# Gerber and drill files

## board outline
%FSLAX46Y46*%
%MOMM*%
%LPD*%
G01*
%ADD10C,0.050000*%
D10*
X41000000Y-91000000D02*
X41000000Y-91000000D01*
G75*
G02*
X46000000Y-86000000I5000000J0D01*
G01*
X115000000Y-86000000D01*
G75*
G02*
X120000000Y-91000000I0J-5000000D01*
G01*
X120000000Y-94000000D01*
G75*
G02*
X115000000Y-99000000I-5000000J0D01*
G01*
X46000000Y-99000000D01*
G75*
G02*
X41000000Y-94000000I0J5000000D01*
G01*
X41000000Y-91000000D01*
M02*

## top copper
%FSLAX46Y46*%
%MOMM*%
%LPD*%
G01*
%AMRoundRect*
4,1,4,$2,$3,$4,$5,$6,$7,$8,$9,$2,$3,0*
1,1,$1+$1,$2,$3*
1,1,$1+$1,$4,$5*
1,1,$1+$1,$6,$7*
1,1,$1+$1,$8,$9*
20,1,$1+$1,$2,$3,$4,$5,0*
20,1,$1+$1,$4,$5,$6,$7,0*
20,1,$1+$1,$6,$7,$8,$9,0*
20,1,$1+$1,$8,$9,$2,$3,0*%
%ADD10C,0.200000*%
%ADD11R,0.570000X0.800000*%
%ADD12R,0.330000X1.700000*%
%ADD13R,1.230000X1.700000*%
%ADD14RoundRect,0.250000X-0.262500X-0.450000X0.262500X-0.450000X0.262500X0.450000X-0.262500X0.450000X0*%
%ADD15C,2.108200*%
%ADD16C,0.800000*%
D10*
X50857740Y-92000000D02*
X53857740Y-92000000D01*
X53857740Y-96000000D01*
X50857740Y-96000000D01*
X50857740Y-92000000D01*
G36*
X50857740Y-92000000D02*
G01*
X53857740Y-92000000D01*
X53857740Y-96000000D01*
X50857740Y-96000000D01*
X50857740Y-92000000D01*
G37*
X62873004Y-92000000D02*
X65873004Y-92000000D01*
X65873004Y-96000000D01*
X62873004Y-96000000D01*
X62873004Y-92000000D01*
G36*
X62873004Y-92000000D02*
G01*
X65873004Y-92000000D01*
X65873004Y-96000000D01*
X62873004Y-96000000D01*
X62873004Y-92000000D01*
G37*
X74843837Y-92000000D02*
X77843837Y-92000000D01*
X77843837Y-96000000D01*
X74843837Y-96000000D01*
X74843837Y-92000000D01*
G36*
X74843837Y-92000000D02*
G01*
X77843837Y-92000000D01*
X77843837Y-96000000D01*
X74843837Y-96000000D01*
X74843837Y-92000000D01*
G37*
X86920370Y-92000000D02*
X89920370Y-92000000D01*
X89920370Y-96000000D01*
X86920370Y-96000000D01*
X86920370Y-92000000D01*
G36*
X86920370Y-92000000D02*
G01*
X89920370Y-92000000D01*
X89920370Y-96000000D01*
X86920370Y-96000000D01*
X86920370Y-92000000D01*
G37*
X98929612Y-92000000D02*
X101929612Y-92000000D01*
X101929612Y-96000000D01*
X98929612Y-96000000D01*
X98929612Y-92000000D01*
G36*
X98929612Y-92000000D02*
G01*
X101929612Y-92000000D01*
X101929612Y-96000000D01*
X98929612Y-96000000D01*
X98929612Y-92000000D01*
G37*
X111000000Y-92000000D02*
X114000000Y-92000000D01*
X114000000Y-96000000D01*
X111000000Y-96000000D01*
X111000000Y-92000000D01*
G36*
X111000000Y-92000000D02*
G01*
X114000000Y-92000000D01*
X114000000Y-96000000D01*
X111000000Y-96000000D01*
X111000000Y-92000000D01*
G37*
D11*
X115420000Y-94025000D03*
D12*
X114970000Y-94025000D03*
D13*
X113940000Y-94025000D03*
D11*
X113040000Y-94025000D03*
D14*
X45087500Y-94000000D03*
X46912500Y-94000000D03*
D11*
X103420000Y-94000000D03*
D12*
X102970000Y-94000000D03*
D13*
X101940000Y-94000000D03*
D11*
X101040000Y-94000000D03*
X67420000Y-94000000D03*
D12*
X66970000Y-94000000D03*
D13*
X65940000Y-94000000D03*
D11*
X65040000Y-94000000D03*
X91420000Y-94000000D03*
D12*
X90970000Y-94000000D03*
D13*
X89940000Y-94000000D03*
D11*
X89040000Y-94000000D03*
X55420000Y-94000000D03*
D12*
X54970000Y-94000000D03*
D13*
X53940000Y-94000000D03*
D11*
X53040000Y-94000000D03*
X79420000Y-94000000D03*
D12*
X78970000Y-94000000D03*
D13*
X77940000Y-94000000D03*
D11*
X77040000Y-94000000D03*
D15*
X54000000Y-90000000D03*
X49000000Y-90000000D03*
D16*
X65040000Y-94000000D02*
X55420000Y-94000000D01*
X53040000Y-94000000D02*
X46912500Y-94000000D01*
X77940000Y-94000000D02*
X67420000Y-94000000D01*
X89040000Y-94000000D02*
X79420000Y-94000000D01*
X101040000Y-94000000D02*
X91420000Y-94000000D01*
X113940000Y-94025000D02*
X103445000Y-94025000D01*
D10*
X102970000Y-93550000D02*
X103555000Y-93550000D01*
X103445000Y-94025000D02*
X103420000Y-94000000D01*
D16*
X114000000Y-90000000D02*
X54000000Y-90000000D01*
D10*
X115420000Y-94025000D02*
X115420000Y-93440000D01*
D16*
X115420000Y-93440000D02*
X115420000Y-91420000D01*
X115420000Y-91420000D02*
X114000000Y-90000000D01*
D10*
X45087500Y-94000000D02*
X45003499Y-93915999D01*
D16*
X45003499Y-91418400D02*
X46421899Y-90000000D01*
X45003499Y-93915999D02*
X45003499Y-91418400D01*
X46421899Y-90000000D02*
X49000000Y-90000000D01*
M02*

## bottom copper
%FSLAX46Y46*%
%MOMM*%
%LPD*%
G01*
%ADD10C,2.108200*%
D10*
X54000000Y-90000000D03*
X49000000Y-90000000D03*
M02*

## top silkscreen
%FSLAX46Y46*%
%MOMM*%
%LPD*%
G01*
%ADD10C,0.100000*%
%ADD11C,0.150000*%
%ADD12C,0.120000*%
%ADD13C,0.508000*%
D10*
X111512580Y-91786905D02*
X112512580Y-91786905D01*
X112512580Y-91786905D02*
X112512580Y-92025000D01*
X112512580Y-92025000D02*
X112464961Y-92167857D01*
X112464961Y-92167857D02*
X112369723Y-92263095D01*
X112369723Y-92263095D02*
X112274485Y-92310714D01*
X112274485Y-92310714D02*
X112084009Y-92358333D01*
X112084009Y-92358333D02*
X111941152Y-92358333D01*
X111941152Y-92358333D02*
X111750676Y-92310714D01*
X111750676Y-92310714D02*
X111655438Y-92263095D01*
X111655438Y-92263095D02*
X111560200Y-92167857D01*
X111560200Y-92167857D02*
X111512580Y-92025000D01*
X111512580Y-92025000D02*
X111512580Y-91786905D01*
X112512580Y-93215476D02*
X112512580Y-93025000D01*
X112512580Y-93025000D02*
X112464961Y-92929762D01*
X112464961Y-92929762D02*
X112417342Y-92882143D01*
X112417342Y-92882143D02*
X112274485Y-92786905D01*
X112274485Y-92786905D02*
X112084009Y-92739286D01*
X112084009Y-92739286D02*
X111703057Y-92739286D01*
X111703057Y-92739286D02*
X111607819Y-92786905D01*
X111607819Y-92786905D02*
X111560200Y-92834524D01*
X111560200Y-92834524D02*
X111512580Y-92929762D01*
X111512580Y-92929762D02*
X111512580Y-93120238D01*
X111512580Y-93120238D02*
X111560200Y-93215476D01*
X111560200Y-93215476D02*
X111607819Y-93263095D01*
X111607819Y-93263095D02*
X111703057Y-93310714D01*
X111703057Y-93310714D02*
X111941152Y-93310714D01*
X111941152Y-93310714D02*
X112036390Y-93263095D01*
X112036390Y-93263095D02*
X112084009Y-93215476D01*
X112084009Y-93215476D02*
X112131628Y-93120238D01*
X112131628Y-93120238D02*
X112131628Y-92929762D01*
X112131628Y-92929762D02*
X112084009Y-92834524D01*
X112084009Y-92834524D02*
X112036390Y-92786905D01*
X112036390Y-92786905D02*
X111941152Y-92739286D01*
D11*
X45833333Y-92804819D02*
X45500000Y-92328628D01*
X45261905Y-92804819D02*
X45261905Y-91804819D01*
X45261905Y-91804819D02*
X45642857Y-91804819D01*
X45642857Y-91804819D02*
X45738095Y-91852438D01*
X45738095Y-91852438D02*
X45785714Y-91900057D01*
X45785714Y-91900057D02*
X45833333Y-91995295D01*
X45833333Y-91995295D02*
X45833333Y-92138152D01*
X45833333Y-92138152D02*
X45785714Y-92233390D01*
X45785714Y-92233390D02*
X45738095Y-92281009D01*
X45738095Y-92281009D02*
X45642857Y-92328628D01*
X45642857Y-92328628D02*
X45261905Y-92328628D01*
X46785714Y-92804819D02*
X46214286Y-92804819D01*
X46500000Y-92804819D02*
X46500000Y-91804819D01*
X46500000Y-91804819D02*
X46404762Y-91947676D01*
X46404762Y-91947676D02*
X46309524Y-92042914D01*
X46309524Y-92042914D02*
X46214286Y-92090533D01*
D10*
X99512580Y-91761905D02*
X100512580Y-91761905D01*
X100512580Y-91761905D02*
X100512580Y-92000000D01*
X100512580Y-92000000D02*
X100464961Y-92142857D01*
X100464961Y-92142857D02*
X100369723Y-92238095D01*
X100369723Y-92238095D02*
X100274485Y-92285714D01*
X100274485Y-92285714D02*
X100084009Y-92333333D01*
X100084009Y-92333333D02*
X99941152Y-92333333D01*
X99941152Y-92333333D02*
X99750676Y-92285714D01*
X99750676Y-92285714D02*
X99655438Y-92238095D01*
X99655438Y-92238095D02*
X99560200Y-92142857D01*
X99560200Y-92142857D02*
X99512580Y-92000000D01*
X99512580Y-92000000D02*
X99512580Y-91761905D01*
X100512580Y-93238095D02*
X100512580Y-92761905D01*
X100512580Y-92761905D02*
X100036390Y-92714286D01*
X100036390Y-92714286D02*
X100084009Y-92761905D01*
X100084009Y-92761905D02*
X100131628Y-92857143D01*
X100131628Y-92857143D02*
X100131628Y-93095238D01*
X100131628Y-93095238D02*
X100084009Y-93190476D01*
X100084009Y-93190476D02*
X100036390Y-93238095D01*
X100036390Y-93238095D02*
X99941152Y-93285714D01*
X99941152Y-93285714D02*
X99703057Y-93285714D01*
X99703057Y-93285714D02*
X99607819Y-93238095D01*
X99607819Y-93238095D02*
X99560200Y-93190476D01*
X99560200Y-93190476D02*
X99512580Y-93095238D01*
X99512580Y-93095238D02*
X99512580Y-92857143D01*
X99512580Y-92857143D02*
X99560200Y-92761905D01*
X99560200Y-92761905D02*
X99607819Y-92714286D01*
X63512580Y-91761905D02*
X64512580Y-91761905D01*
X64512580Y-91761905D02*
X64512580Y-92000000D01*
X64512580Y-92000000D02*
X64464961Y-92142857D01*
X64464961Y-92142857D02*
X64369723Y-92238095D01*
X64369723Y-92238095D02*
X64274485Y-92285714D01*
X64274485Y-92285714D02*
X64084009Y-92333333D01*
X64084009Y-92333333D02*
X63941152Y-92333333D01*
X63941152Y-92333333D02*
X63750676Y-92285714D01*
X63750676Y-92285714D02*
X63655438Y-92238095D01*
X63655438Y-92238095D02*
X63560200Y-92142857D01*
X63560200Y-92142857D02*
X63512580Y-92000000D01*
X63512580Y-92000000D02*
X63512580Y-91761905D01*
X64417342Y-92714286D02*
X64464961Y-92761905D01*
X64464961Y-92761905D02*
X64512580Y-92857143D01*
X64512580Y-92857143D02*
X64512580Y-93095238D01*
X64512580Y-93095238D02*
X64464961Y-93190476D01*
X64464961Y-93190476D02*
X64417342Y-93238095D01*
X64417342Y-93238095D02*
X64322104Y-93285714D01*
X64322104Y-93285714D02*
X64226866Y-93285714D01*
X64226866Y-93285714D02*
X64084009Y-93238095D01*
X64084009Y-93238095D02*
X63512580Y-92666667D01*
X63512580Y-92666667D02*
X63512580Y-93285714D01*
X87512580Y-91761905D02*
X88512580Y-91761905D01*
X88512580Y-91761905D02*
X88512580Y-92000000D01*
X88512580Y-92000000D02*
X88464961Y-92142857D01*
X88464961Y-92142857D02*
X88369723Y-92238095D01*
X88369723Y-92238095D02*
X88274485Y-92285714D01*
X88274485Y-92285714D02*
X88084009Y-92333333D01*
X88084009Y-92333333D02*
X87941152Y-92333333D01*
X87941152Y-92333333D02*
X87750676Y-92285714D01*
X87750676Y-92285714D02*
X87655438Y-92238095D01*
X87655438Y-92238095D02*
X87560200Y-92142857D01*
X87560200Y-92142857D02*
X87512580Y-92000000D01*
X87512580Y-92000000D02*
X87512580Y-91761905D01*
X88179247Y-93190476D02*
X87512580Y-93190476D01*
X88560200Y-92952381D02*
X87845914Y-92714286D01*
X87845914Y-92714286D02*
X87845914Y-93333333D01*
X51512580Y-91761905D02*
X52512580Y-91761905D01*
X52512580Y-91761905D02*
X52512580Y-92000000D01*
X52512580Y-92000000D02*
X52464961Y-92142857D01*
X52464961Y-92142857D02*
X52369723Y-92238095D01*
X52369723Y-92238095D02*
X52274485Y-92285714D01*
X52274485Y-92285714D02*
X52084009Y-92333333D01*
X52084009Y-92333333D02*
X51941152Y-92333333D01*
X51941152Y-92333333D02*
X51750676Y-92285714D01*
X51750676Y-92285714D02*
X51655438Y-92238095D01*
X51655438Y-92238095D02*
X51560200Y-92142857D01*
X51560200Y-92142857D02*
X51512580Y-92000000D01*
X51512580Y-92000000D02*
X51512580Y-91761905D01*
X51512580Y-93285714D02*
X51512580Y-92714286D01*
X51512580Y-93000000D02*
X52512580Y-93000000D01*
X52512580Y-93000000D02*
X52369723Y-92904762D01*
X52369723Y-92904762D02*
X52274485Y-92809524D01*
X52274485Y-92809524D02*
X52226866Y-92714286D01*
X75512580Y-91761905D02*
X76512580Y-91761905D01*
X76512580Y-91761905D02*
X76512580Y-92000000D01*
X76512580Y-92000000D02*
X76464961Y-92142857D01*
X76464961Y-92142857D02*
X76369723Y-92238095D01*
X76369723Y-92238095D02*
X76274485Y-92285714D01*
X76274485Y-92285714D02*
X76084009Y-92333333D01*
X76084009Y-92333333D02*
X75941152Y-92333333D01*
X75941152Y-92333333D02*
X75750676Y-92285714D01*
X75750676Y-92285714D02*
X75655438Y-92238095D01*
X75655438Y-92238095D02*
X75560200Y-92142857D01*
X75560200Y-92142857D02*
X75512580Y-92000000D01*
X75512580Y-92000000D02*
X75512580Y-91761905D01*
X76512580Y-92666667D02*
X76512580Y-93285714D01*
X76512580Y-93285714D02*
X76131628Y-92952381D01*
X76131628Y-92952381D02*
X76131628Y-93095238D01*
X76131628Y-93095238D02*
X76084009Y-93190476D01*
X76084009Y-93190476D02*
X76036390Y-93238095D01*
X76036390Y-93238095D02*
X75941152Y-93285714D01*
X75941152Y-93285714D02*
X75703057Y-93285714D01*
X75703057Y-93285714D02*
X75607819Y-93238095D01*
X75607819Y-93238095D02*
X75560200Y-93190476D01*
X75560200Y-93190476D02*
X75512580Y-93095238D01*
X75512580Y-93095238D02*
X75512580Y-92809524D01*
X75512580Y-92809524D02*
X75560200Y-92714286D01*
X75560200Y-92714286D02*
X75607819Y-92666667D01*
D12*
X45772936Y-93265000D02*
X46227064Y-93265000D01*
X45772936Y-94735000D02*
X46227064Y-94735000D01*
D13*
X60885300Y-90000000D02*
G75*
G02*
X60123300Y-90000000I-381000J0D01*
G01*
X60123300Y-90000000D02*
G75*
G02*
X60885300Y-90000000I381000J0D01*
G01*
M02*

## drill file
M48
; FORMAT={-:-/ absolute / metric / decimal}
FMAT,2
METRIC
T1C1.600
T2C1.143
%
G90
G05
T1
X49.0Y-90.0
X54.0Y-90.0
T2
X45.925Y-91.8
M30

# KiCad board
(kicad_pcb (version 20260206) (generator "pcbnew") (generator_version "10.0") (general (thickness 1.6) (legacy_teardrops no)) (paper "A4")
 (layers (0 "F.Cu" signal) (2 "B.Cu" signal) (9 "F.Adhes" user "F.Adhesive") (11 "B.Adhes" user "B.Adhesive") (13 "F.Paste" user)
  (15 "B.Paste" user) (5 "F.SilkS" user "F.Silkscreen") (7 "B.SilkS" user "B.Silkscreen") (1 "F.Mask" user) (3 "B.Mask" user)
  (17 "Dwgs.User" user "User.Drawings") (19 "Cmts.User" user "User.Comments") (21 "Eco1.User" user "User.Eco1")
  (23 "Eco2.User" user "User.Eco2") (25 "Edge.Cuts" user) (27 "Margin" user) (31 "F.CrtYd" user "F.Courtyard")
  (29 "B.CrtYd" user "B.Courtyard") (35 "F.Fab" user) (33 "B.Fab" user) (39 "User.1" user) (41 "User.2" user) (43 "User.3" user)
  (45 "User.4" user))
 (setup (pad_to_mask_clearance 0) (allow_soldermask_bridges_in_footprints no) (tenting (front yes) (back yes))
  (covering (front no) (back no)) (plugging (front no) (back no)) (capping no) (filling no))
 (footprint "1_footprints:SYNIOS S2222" (layer "F.Cu") (at 114.97 94.025 -90)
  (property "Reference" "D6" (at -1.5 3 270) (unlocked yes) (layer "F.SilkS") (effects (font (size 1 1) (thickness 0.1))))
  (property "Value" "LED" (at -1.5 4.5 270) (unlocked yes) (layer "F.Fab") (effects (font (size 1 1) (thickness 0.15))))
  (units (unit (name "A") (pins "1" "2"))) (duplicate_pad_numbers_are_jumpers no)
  (pad "1" smd rect (at 0 -0.45 270) (size 0.8 0.57) (layers "F.Cu" "F.Mask" "F.Paste") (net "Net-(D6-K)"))
  (pad "1" smd rect (at 0 0 270) (size 1.7 0.33) (layers "F.Cu" "F.Mask" "F.Paste") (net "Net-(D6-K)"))
  (pad "2" smd rect (at 0 1.03 270) (size 1.7 1.23) (layers "F.Cu" "F.Mask" "F.Paste") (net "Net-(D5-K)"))
  (pad "2" smd rect (at 0 1.93 270) (size 0.8 0.57) (layers "F.Cu" "F.Mask" "F.Paste") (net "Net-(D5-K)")))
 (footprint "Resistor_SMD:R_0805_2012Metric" (layer "F.Cu") (at 46 94)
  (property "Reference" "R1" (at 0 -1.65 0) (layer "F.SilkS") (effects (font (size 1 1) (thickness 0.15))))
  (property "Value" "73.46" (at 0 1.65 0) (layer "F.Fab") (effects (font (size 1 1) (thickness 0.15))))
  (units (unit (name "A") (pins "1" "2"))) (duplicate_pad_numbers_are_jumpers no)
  (fp_line (start -0.227064 -0.735) (end 0.227064 -0.735) (stroke (width 0.12) (type solid)) (layer "F.SilkS"))
  (fp_line (start -0.227064 0.735) (end 0.227064 0.735) (stroke (width 0.12) (type solid)) (layer "F.SilkS"))
  (pad "1" smd roundrect (at -0.9125 0) (size 1.025 1.4) (layers "F.Cu" "F.Mask" "F.Paste") (roundrect_rratio 0.243902)
   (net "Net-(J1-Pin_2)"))
  (pad "2" smd roundrect (at 0.9125 0) (size 1.025 1.4) (layers "F.Cu" "F.Mask" "F.Paste") (roundrect_rratio 0.243902) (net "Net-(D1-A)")))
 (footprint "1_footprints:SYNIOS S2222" (layer "F.Cu") (at 102.97 94 -90)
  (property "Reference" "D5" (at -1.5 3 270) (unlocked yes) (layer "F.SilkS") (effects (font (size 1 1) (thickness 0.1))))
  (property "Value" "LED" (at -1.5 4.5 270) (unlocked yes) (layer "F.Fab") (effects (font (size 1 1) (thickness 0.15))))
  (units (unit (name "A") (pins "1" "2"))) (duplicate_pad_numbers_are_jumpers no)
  (pad "1" smd rect (at 0 -0.45 270) (size 0.8 0.57) (layers "F.Cu" "F.Mask" "F.Paste") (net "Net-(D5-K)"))
  (pad "1" smd rect (at 0 0 270) (size 1.7 0.33) (layers "F.Cu" "F.Mask" "F.Paste") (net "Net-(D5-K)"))
  (pad "2" smd rect (at 0 1.03 270) (size 1.7 1.23) (layers "F.Cu" "F.Mask" "F.Paste") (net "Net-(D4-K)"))
  (pad "2" smd rect (at 0 1.93 270) (size 0.8 0.57) (layers "F.Cu" "F.Mask" "F.Paste") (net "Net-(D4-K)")))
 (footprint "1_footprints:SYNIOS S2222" (layer "F.Cu") (at 66.97 94 -90)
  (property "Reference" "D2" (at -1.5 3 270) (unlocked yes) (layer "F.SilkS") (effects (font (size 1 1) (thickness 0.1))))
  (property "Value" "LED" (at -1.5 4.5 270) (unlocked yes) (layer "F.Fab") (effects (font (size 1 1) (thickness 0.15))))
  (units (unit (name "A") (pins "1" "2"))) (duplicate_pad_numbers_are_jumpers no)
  (pad "1" smd rect (at 0 -0.45 270) (size 0.8 0.57) (layers "F.Cu" "F.Mask" "F.Paste") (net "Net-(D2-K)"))
  (pad "1" smd rect (at 0 0 270) (size 1.7 0.33) (layers "F.Cu" "F.Mask" "F.Paste") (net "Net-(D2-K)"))
  (pad "2" smd rect (at 0 1.03 270) (size 1.7 1.23) (layers "F.Cu" "F.Mask" "F.Paste") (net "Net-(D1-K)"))
  (pad "2" smd rect (at 0 1.93 270) (size 0.8 0.57) (layers "F.Cu" "F.Mask" "F.Paste") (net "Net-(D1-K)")))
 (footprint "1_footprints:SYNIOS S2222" (layer "F.Cu") (at 90.97 94 -90)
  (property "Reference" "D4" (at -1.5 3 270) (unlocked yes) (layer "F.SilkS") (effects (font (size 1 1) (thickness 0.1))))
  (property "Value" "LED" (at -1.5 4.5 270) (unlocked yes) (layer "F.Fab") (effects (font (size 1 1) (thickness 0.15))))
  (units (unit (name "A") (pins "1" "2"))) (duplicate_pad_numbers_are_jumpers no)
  (pad "1" smd rect (at 0 -0.45 270) (size 0.8 0.57) (layers "F.Cu" "F.Mask" "F.Paste") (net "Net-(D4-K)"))
  (pad "1" smd rect (at 0 0 270) (size 1.7 0.33) (layers "F.Cu" "F.Mask" "F.Paste") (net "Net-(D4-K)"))
  (pad "2" smd rect (at 0 1.03 270) (size 1.7 1.23) (layers "F.Cu" "F.Mask" "F.Paste") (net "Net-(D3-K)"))
  (pad "2" smd rect (at 0 1.93 270) (size 0.8 0.57) (layers "F.Cu" "F.Mask" "F.Paste") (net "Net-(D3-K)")))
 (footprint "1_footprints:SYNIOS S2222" (layer "F.Cu") (at 54.97 94 -90)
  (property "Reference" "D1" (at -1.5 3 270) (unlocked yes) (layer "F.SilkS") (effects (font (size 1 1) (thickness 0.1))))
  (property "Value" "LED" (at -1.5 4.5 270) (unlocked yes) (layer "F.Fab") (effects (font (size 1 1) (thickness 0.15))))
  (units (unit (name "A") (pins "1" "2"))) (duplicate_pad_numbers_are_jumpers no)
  (pad "1" smd rect (at 0 -0.45 270) (size 0.8 0.57) (layers "F.Cu" "F.Mask" "F.Paste") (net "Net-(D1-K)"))
  (pad "1" smd rect (at 0 0 270) (size 1.7 0.33) (layers "F.Cu" "F.Mask" "F.Paste") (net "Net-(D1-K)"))
  (pad "2" smd rect (at 0 1.03 270) (size 1.7 1.23) (layers "F.Cu" "F.Mask" "F.Paste") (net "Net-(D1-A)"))
  (pad "2" smd rect (at 0 1.93 270) (size 0.8 0.57) (layers "F.Cu" "F.Mask" "F.Paste") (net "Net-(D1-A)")))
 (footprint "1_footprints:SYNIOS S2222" (layer "F.Cu") (at 78.97 94 -90)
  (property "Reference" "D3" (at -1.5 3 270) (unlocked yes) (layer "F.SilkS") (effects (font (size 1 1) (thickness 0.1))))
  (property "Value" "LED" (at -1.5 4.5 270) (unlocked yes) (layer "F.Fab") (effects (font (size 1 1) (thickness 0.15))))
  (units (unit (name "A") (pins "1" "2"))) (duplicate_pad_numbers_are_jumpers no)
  (pad "1" smd rect (at 0 -0.45 270) (size 0.8 0.57) (layers "F.Cu" "F.Mask" "F.Paste") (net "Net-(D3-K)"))
  (pad "1" smd rect (at 0 0 270) (size 1.7 0.33) (layers "F.Cu" "F.Mask" "F.Paste") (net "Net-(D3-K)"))
  (pad "2" smd rect (at 0 1.03 270) (size 1.7 1.23) (layers "F.Cu" "F.Mask" "F.Paste") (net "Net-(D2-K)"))
  (pad "2" smd rect (at 0 1.93 270) (size 0.8 0.57) (layers "F.Cu" "F.Mask" "F.Paste") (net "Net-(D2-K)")))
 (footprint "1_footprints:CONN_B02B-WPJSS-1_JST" (layer "B.Cu") (at 54 90 180)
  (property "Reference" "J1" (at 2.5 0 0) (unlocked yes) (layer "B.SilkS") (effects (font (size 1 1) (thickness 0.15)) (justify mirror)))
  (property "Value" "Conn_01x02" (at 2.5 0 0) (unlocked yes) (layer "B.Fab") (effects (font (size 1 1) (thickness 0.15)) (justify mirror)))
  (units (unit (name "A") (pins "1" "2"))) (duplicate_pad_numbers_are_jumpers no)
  (fp_circle (center -6.5043 0) (end -6.1233 0) (stroke (width 0.508) (type solid)) (fill no) (layer "F.SilkS"))
  (pad "" np_thru_hole circle (at 8.075001 -1.800098 180) (size 1.143 1.143) (drill 1.143) (layers))
  (pad "1" thru_hole circle (at 0 0 180) (size 2.1082 2.1082) (drill 1.6002) (layers "*.Cu" "*.Mask") (remove_unused_layers no)
   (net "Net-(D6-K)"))
  (pad "2" thru_hole circle (at 5 0 180) (size 2.1082 2.1082) (drill 1.6002) (layers "*.Cu" "*.Mask") (remove_unused_layers no)
   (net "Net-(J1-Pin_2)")))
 (gr_rect (start 50.85774 92) (end 53.85774 96) (stroke (width 0.2) (type solid)) (fill yes) (layer "F.Cu") (net "Net-(D1-A)"))
 (gr_rect (start 62.873004 92) (end 65.873004 96) (stroke (width 0.2) (type solid)) (fill yes) (layer "F.Cu") (net "Net-(D1-K)"))
 (gr_rect (start 74.843837 92) (end 77.843837 96) (stroke (width 0.2) (type solid)) (fill yes) (layer "F.Cu") (net "Net-(D2-K)"))
 (gr_rect (start 86.92037 92) (end 89.92037 96) (stroke (width 0.2) (type solid)) (fill yes) (layer "F.Cu") (net "Net-(D3-K)"))
 (gr_rect (start 98.929612 92) (end 101.929612 96) (stroke (width 0.2) (type solid)) (fill yes) (layer "F.Cu") (net "Net-(D4-K)"))
 (gr_rect (start 111 92) (end 114 96) (stroke (width 0.2) (type solid)) (fill yes) (layer "F.Cu") (net "Net-(D5-K)"))
 (gr_rect (start 41 86) (end 120 99) (radius 5) (stroke (width 0.05) (type solid)) (fill no) (layer "Edge.Cuts"))
 (segment (start 65.04 94) (end 55.42 94) (width 0.8) (layer "F.Cu") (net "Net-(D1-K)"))
 (segment (start 53.04 94) (end 46.9125 94) (width 0.8) (layer "F.Cu") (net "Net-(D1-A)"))
 (segment (start 77.94 94) (end 67.42 94) (width 0.8) (layer "F.Cu") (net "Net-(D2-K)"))
 (segment (start 89.04 94) (end 79.42 94) (width 0.8) (layer "F.Cu") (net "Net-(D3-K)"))
 (segment (start 101.04 94) (end 91.42 94) (width 0.8) (layer "F.Cu") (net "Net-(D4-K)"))
 (segment (start 113.94 94.025) (end 103.445 94.025) (width 0.8) (layer "F.Cu") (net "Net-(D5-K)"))
 (segment (start 102.97 93.55) (end 103.555 93.55) (width 0.2) (layer "F.Cu") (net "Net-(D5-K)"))
 (segment (start 103.445 94.025) (end 103.42 94) (width 0.2) (layer "F.Cu") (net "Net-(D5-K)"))
 (segment (start 114 90) (end 54 90) (width 0.8) (layer "F.Cu") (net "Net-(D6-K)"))
 (segment (start 115.42 94.025) (end 115.42 93.44) (width 0.2) (layer "F.Cu") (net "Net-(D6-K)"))
 (segment (start 115.42 93.44) (end 115.42 91.42) (width 0.8) (layer "F.Cu") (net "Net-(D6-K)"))
 (segment (start 115.42 91.42) (end 114 90) (width 0.8) (layer "F.Cu") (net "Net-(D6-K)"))
 (segment (start 45.0875 94) (end 45.003499 93.915999) (width 0.2) (layer "F.Cu") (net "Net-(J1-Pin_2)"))
 (segment (start 45.003499 91.4184) (end 46.421899 90) (width 0.8) (layer "F.Cu") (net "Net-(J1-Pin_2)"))
 (segment (start 45.003499 93.915999) (end 45.003499 91.4184) (width 0.8) (layer "F.Cu") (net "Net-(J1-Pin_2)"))
 (segment (start 46.421899 90) (end 49 90) (width 0.8) (layer "F.Cu") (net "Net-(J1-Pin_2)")))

